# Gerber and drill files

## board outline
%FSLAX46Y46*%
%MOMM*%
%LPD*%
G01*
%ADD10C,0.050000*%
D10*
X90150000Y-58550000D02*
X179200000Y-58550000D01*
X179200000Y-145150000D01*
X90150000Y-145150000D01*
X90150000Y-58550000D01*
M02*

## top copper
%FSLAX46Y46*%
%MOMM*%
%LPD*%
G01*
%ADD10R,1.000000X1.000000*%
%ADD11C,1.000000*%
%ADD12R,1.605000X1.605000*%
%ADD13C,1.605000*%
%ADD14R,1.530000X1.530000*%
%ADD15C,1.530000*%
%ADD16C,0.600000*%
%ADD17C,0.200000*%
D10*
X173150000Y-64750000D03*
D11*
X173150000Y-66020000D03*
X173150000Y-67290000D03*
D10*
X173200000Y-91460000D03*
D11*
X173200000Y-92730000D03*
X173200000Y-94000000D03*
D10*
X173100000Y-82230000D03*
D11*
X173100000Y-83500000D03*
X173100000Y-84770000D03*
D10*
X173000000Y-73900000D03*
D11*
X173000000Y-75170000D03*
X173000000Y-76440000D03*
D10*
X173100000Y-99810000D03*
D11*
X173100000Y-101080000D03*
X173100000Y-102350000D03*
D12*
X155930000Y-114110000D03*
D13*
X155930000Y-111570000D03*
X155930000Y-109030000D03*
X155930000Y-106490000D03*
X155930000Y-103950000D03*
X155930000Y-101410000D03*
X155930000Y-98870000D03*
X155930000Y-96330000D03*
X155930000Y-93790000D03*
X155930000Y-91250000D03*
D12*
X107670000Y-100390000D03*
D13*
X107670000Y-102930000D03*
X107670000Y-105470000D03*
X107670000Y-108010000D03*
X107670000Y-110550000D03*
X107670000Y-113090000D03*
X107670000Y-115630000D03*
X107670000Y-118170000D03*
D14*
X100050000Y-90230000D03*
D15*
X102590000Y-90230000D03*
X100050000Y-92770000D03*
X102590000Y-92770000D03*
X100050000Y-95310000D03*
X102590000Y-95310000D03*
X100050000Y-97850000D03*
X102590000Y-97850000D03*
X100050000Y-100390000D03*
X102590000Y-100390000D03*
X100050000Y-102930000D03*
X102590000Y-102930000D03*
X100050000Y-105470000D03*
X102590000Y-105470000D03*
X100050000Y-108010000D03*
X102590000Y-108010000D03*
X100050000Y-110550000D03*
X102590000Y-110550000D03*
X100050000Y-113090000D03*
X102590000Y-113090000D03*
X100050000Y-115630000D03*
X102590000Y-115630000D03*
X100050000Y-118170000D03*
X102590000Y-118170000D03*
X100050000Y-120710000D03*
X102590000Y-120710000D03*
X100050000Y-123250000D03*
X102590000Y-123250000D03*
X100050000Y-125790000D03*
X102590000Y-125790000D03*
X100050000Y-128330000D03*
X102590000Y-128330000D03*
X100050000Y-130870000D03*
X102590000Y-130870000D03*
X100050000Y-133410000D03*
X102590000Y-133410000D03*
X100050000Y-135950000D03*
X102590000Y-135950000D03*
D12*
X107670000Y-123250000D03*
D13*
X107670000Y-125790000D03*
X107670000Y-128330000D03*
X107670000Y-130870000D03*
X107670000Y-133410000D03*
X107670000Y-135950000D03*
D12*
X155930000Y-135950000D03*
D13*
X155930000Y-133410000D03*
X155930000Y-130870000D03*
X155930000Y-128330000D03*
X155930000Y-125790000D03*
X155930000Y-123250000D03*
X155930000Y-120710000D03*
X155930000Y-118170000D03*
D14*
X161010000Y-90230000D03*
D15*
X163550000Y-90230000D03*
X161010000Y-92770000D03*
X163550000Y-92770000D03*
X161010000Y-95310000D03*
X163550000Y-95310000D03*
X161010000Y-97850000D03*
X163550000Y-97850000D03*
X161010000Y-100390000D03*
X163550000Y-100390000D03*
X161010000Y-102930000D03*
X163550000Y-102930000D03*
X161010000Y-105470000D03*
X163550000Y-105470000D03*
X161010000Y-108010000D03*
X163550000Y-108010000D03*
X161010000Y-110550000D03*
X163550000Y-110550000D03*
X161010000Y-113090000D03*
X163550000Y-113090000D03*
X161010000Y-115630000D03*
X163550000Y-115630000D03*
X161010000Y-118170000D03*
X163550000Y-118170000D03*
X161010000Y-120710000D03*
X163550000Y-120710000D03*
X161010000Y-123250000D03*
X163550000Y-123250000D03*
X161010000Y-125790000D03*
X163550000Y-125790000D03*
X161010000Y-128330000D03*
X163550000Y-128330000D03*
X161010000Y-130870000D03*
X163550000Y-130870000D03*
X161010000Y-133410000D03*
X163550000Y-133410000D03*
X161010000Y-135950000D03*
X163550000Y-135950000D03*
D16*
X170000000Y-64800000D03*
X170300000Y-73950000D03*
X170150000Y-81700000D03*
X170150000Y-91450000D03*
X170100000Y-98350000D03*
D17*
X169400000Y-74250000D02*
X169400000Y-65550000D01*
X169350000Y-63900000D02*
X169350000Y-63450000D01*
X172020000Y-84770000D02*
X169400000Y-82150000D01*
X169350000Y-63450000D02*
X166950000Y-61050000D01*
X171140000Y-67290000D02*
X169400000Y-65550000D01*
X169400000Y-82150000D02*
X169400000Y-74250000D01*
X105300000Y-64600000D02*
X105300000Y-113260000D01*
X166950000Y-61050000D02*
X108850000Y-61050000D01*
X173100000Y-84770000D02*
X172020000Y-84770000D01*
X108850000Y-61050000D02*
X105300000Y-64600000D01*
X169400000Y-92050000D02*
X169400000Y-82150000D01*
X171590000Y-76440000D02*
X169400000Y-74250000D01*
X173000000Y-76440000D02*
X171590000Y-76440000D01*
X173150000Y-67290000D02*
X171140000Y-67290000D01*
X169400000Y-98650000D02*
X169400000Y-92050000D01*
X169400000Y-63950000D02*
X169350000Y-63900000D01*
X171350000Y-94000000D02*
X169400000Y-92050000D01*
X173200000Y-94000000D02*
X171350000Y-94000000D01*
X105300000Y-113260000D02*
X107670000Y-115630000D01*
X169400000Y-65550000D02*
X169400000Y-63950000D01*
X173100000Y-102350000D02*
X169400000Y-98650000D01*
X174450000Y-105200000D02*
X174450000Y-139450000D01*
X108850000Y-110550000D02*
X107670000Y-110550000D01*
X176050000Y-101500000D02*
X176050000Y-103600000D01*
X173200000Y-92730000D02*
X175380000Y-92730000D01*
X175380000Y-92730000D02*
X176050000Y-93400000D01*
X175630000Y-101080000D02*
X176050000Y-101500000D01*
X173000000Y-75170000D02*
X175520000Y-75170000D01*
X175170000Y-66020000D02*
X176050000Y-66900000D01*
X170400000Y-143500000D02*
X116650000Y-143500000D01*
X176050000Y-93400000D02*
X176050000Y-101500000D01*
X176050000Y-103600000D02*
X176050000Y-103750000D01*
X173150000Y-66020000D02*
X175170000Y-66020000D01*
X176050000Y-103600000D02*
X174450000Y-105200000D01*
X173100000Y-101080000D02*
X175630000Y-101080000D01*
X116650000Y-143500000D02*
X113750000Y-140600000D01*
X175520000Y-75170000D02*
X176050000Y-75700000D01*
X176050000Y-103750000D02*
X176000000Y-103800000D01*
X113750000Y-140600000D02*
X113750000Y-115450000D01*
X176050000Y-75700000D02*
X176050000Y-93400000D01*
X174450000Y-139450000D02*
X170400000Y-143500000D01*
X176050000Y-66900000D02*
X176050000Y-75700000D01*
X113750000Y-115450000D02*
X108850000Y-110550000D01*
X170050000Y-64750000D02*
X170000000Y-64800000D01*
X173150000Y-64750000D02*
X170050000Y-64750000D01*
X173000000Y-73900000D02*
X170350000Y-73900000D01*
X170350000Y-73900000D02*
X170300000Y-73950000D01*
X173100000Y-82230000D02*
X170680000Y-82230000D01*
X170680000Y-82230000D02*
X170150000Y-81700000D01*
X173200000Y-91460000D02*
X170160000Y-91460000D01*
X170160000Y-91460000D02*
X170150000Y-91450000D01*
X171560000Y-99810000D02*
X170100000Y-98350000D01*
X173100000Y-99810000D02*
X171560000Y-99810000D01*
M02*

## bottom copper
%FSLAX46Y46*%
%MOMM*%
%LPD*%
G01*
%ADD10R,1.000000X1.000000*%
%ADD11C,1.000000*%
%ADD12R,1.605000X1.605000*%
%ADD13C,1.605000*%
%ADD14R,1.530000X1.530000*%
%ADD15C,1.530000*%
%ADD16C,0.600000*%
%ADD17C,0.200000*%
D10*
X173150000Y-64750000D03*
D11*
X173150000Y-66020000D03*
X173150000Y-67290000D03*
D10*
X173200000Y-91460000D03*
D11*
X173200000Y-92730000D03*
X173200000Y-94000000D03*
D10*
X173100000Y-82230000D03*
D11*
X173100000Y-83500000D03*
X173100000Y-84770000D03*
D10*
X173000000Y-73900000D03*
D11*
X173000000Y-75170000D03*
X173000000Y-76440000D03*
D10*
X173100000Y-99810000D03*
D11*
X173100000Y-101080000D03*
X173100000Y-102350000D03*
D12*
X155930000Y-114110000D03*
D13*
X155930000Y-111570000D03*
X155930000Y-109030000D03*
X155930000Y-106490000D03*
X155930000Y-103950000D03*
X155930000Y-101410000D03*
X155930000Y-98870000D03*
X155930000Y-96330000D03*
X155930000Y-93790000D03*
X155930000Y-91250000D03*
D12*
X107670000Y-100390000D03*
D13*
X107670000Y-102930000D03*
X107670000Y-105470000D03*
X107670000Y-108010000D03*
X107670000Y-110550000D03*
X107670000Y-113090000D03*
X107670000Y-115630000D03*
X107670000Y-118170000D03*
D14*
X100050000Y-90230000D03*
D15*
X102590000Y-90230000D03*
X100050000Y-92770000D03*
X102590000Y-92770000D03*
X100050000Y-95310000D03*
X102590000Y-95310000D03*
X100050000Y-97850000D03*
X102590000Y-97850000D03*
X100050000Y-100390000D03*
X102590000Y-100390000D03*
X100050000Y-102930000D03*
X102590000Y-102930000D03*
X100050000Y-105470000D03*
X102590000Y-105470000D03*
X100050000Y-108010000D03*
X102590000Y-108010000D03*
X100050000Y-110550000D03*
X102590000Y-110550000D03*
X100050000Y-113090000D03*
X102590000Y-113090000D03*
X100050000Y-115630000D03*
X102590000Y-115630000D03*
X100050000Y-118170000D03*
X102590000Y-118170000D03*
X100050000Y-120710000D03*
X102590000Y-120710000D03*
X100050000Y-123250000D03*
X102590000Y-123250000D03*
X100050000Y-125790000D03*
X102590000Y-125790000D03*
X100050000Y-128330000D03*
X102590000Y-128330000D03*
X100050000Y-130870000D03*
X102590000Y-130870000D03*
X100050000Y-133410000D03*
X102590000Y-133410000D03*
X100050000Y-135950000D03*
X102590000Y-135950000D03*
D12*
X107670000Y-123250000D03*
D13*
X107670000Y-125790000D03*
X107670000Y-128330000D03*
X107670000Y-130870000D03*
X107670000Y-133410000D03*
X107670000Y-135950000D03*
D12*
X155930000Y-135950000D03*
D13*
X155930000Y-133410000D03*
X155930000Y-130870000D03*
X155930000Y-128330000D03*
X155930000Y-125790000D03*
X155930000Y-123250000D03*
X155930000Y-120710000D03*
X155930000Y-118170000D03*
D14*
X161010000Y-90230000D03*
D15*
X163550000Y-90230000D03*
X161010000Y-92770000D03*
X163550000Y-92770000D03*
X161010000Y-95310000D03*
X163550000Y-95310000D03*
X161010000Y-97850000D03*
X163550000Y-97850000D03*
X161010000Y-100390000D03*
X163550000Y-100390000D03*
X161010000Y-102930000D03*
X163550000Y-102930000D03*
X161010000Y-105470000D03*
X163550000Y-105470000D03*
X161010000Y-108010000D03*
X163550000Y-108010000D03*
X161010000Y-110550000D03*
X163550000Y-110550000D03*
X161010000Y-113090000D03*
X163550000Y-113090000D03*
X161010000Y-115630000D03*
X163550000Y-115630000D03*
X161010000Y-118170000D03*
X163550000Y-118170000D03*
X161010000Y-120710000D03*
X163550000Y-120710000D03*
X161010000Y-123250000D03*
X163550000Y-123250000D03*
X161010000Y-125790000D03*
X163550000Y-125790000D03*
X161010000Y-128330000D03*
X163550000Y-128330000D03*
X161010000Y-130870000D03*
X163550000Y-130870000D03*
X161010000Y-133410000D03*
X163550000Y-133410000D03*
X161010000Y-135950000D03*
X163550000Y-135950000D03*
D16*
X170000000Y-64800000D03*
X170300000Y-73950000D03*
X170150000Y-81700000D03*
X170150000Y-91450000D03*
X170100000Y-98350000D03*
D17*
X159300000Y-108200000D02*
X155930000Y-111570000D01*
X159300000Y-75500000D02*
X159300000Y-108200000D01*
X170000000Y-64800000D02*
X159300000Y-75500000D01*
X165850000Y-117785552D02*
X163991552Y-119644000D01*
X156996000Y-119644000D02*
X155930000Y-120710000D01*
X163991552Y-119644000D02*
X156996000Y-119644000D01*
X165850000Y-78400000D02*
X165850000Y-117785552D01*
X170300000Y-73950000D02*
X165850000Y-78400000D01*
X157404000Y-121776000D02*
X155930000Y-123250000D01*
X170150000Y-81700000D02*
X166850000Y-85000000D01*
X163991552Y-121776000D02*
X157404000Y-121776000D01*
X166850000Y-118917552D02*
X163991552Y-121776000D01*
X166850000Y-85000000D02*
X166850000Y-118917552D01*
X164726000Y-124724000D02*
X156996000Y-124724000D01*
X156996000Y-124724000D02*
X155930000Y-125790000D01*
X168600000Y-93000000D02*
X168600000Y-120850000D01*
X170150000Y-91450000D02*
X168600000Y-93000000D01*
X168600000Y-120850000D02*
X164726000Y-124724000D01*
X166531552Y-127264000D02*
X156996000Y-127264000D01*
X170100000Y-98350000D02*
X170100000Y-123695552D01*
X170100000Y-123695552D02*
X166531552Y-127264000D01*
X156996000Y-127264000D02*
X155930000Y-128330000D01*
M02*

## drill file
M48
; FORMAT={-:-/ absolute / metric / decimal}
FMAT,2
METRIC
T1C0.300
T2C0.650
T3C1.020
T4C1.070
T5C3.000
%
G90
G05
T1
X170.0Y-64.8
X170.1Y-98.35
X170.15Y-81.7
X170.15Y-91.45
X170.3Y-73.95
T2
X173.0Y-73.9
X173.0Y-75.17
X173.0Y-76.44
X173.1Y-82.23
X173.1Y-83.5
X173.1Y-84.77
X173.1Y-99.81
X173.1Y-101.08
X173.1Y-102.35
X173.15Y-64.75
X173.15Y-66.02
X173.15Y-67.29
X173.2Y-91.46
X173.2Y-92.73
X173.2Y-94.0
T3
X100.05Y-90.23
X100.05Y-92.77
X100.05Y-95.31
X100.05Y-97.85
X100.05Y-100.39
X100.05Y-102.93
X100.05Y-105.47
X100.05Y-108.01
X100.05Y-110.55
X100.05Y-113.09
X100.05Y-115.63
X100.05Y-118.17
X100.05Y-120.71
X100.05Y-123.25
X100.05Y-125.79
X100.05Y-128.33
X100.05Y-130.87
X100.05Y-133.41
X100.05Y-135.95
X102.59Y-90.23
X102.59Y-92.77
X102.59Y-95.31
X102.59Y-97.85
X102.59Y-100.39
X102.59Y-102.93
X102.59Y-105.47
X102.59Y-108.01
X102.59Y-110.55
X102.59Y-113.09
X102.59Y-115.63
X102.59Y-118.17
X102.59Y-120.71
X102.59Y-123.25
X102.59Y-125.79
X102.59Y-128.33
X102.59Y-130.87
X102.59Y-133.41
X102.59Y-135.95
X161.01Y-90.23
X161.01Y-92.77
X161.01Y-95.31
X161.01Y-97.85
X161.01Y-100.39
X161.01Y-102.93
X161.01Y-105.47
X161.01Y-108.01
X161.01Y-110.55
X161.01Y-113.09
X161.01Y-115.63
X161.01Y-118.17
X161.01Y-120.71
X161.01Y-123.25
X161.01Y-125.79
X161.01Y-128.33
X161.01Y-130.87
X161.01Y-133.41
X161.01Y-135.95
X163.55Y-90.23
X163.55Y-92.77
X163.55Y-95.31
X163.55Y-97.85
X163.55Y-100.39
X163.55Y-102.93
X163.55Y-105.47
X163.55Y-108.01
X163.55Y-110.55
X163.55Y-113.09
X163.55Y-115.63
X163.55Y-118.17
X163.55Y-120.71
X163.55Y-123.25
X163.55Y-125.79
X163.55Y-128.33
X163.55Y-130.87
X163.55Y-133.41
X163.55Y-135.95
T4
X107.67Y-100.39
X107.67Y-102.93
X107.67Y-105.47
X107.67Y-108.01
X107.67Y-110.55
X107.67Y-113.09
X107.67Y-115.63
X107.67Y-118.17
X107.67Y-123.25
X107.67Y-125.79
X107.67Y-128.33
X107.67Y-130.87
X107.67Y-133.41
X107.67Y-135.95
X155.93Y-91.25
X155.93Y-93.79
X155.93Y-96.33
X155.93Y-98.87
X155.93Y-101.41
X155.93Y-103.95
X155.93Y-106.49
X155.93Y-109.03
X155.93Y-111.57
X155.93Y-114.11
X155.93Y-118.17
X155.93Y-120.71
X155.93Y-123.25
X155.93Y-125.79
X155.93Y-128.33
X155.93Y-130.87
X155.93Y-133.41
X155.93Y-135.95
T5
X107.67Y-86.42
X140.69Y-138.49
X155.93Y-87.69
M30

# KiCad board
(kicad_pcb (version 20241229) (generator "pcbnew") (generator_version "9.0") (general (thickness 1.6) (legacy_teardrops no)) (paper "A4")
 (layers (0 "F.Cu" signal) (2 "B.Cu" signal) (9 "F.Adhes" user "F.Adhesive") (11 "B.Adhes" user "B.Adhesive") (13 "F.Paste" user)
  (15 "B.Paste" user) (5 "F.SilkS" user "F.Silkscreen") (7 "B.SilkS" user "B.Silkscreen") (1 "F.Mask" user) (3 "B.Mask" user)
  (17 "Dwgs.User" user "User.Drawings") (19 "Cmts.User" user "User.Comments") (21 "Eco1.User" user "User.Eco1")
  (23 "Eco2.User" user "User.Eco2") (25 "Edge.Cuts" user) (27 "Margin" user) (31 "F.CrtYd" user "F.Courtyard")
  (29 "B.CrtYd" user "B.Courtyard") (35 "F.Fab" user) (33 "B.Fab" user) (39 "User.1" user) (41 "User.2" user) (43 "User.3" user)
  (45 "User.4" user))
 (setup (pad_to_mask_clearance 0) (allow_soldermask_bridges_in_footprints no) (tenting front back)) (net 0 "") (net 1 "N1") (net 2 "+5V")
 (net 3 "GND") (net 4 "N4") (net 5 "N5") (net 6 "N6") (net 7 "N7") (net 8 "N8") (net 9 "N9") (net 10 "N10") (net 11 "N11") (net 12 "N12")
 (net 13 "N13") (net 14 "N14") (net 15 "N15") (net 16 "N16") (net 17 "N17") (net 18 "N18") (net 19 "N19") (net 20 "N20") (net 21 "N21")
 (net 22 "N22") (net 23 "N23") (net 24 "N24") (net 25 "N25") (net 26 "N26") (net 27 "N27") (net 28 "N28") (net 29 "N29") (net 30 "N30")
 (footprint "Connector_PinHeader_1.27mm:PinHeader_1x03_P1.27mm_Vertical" (layer "F.Cu") (at 173.15 64.75)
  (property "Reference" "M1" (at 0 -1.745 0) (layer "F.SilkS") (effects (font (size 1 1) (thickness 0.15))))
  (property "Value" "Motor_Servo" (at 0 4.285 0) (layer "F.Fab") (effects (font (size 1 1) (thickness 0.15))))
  (pad "1" thru_hole rect (at 0 0) (size 1 1) (drill 0.65) (layers "*.Cu" "*.Mask") (remove_unused_layers no) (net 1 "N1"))
  (pad "2" thru_hole circle (at 0 1.27) (size 1 1) (drill 0.65) (layers "*.Cu" "*.Mask") (remove_unused_layers no) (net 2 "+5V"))
  (pad "3" thru_hole circle (at 0 2.54) (size 1 1) (drill 0.65) (layers "*.Cu" "*.Mask") (remove_unused_layers no) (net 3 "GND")))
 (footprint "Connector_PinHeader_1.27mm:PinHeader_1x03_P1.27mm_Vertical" (layer "F.Cu") (at 173.2 91.46)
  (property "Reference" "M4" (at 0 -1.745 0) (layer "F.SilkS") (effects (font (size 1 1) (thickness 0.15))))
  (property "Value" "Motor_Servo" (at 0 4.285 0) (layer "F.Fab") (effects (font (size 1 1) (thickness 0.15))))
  (pad "1" thru_hole rect (at 0 0) (size 1 1) (drill 0.65) (layers "*.Cu" "*.Mask") (remove_unused_layers no) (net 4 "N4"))
  (pad "2" thru_hole circle (at 0 1.27) (size 1 1) (drill 0.65) (layers "*.Cu" "*.Mask") (remove_unused_layers no) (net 2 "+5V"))
  (pad "3" thru_hole circle (at 0 2.54) (size 1 1) (drill 0.65) (layers "*.Cu" "*.Mask") (remove_unused_layers no) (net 3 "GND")))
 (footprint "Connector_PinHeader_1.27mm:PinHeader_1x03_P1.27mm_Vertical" (layer "F.Cu") (at 173.1 82.23)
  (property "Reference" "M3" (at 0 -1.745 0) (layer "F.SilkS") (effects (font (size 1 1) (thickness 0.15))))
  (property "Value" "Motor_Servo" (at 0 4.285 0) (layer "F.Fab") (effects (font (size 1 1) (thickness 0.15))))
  (pad "1" thru_hole rect (at 0 0) (size 1 1) (drill 0.65) (layers "*.Cu" "*.Mask") (remove_unused_layers no) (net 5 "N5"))
  (pad "2" thru_hole circle (at 0 1.27) (size 1 1) (drill 0.65) (layers "*.Cu" "*.Mask") (remove_unused_layers no) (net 2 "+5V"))
  (pad "3" thru_hole circle (at 0 2.54) (size 1 1) (drill 0.65) (layers "*.Cu" "*.Mask") (remove_unused_layers no) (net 3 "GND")))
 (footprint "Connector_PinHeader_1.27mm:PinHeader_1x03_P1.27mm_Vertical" (layer "F.Cu") (at 173 73.9)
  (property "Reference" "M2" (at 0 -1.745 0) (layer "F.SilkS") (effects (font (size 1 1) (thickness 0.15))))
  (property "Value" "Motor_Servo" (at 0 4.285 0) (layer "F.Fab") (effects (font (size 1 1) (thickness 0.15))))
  (pad "1" thru_hole rect (at 0 0) (size 1 1) (drill 0.65) (layers "*.Cu" "*.Mask") (remove_unused_layers no) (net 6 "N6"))
  (pad "2" thru_hole circle (at 0 1.27) (size 1 1) (drill 0.65) (layers "*.Cu" "*.Mask") (remove_unused_layers no) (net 2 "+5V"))
  (pad "3" thru_hole circle (at 0 2.54) (size 1 1) (drill 0.65) (layers "*.Cu" "*.Mask") (remove_unused_layers no) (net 3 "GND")))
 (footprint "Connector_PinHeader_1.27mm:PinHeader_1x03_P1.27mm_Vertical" (layer "F.Cu") (at 173.1 99.81)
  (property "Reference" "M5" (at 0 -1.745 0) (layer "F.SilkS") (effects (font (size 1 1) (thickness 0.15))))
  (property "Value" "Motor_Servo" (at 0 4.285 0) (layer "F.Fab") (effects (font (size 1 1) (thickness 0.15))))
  (pad "1" thru_hole rect (at 0 0) (size 1 1) (drill 0.65) (layers "*.Cu" "*.Mask") (remove_unused_layers no) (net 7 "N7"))
  (pad "2" thru_hole circle (at 0 1.27) (size 1 1) (drill 0.65) (layers "*.Cu" "*.Mask") (remove_unused_layers no) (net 2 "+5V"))
  (pad "3" thru_hole circle (at 0 2.54) (size 1 1) (drill 0.65) (layers "*.Cu" "*.Mask") (remove_unused_layers no) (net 3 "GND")))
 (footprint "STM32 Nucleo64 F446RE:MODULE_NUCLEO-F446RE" (layer "F.Cu") (at 131.8 99.74)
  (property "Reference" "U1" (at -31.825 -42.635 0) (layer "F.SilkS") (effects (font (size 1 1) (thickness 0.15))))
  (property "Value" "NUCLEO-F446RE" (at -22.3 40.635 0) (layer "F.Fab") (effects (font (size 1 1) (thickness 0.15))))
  (pad "" np_thru_hole circle (at -24.13 -13.32) (size 3 3) (drill 3) (layers "*.Cu" "*.Mask"))
  (pad "" np_thru_hole circle (at 8.89 38.75) (size 3 3) (drill 3) (layers "*.Cu" "*.Mask"))
  (pad "" np_thru_hole circle (at 24.13 -12.05) (size 3 3) (drill 3) (layers "*.Cu" "*.Mask"))
  (pad "CN5_1" thru_hole rect (at 24.13 14.37) (size 1.605 1.605) (drill 1.07) (layers "*.Cu" "*.Mask") (remove_unused_layers no)
   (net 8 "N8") (solder_mask_margin 0.102))
  (pad "CN5_2" thru_hole circle (at 24.13 11.83) (size 1.605 1.605) (drill 1.07) (layers "*.Cu" "*.Mask") (remove_unused_layers no)
   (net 1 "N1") (solder_mask_margin 0.102))
  (pad "CN5_3" thru_hole circle (at 24.13 9.29) (size 1.605 1.605) (drill 1.07) (layers "*.Cu" "*.Mask") (remove_unused_layers no)
   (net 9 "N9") (solder_mask_margin 0.102))
  (pad "CN5_4" thru_hole circle (at 24.13 6.75) (size 1.605 1.605) (drill 1.07) (layers "*.Cu" "*.Mask") (remove_unused_layers no)
   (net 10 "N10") (solder_mask_margin 0.102))
  (pad "CN5_5" thru_hole circle (at 24.13 4.21) (size 1.605 1.605) (drill 1.07) (layers "*.Cu" "*.Mask") (remove_unused_layers no)
   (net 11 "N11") (solder_mask_margin 0.102))
  (pad "CN5_6" thru_hole circle (at 24.13 1.67) (size 1.605 1.605) (drill 1.07) (layers "*.Cu" "*.Mask") (remove_unused_layers no)
   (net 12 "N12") (solder_mask_margin 0.102))
  (pad "CN5_7" thru_hole circle (at 24.13 -0.87) (size 1.605 1.605) (drill 1.07) (layers "*.Cu" "*.Mask") (remove_unused_layers no)
   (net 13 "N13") (solder_mask_margin 0.102))
  (pad "CN5_8" thru_hole circle (at 24.13 -3.41) (size 1.605 1.605) (drill 1.07) (layers "*.Cu" "*.Mask") (remove_unused_layers no)
   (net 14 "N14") (solder_mask_margin 0.102))
  (pad "CN5_9" thru_hole circle (at 24.13 -5.95) (size 1.605 1.605) (drill 1.07) (layers "*.Cu" "*.Mask") (remove_unused_layers no)
   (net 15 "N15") (solder_mask_margin 0.102))
  (pad "CN5_10" thru_hole circle (at 24.13 -8.49) (size 1.605 1.605) (drill 1.07) (layers "*.Cu" "*.Mask") (remove_unused_layers no)
   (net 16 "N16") (solder_mask_margin 0.102))
  (pad "CN6_1" thru_hole rect (at -24.13 0.65) (size 1.605 1.605) (drill 1.07) (layers "*.Cu" "*.Mask") (remove_unused_layers no)
   (solder_mask_margin 0.102))
  (pad "CN6_2" thru_hole circle (at -24.13 3.19) (size 1.605 1.605) (drill 1.07) (layers "*.Cu" "*.Mask") (remove_unused_layers no)
   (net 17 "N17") (solder_mask_margin 0.102))
  (pad "CN6_3" thru_hole circle (at -24.13 5.73) (size 1.605 1.605) (drill 1.07) (layers "*.Cu" "*.Mask") (remove_unused_layers no)
   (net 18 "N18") (solder_mask_margin 0.102))
  (pad "CN6_4" thru_hole circle (at -24.13 8.27) (size 1.605 1.605) (drill 1.07) (layers "*.Cu" "*.Mask") (remove_unused_layers no)
   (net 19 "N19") (solder_mask_margin 0.102))
  (pad "CN6_5" thru_hole circle (at -24.13 10.81) (size 1.605 1.605) (drill 1.07) (layers "*.Cu" "*.Mask") (remove_unused_layers no)
   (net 2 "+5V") (solder_mask_margin 0.102))
  (pad "CN6_6" thru_hole circle (at -24.13 13.35) (size 1.605 1.605) (drill 1.07) (layers "*.Cu" "*.Mask") (remove_unused_layers no)
   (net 3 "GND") (solder_mask_margin 0.102))
  (pad "CN6_7" thru_hole circle (at -24.13 15.89) (size 1.605 1.605) (drill 1.07) (layers "*.Cu" "*.Mask") (remove_unused_layers no)
   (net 3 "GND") (solder_mask_margin 0.102))
  (pad "CN6_8" thru_hole circle (at -24.13 18.43) (size 1.605 1.605) (drill 1.07) (layers "*.Cu" "*.Mask") (remove_unused_layers no)
   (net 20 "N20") (solder_mask_margin 0.102))
  (pad "CN7_1" thru_hole rect (at -31.75 -9.51) (size 1.53 1.53) (drill 1.02) (layers "*.Cu" "*.Mask") (remove_unused_layers no)
   (solder_mask_margin 0.102))
  (pad "CN7_2" thru_hole circle (at -29.21 -9.51) (size 1.53 1.53) (drill 1.02) (layers "*.Cu" "*.Mask") (remove_unused_layers no)
   (solder_mask_margin 0.102))
  (pad "CN7_3" thru_hole circle (at -31.75 -6.97) (size 1.53 1.53) (drill 1.02) (layers "*.Cu" "*.Mask") (remove_unused_layers no)
   (solder_mask_margin 0.102))
  (pad "CN7_4" thru_hole circle (at -29.21 -6.97) (size 1.53 1.53) (drill 1.02) (layers "*.Cu" "*.Mask") (remove_unused_layers no)
   (solder_mask_margin 0.102))
  (pad "CN7_5" thru_hole circle (at -31.75 -4.43) (size 1.53 1.53) (drill 1.02) (layers "*.Cu" "*.Mask") (remove_unused_layers no)
   (solder_mask_margin 0.102))
  (pad "CN7_6" thru_hole circle (at -29.21 -4.43) (size 1.53 1.53) (drill 1.02) (layers "*.Cu" "*.Mask") (remove_unused_layers no)
   (solder_mask_margin 0.102))
  (pad "CN7_7" thru_hole circle (at -31.75 -1.89) (size 1.53 1.53) (drill 1.02) (layers "*.Cu" "*.Mask") (remove_unused_layers no)
   (solder_mask_margin 0.102))
  (pad "CN7_8" thru_hole circle (at -29.21 -1.89) (size 1.53 1.53) (drill 1.02) (layers "*.Cu" "*.Mask") (remove_unused_layers no)
   (solder_mask_margin 0.102))
  (pad "CN7_9" thru_hole circle (at -31.75 0.65) (size 1.53 1.53) (drill 1.02) (layers "*.Cu" "*.Mask") (remove_unused_layers no)
   (solder_mask_margin 0.102))
  (pad "CN7_10" thru_hole circle (at -29.21 0.65) (size 1.53 1.53) (drill 1.02) (layers "*.Cu" "*.Mask") (remove_unused_layers no)
   (solder_mask_margin 0.102))
  (pad "CN7_11" thru_hole circle (at -31.75 3.19) (size 1.53 1.53) (drill 1.02) (layers "*.Cu" "*.Mask") (remove_unused_layers no)
   (solder_mask_margin 0.102))
  (pad "CN7_12" thru_hole circle (at -29.21 3.19) (size 1.53 1.53) (drill 1.02) (layers "*.Cu" "*.Mask") (remove_unused_layers no)
   (solder_mask_margin 0.102))
  (pad "CN7_13" thru_hole circle (at -31.75 5.73) (size 1.53 1.53) (drill 1.02) (layers "*.Cu" "*.Mask") (remove_unused_layers no)
   (solder_mask_margin 0.102))
  (pad "CN7_14" thru_hole circle (at -29.21 5.73) (size 1.53 1.53) (drill 1.02) (layers "*.Cu" "*.Mask") (remove_unused_layers no)
   (solder_mask_margin 0.102))
  (pad "CN7_15" thru_hole circle (at -31.75 8.27) (size 1.53 1.53) (drill 1.02) (layers "*.Cu" "*.Mask") (remove_unused_layers no)
   (solder_mask_margin 0.102))
  (pad "CN7_16" thru_hole circle (at -29.21 8.27) (size 1.53 1.53) (drill 1.02) (layers "*.Cu" "*.Mask") (remove_unused_layers no)
   (solder_mask_margin 0.102))
  (pad "CN7_17" thru_hole circle (at -31.75 10.81) (size 1.53 1.53) (drill 1.02) (layers "*.Cu" "*.Mask") (remove_unused_layers no)
   (solder_mask_margin 0.102))
  (pad "CN7_18" thru_hole circle (at -29.21 10.81) (size 1.53 1.53) (drill 1.02) (layers "*.Cu" "*.Mask") (remove_unused_layers no)
   (solder_mask_margin 0.102))
  (pad "CN7_19" thru_hole circle (at -31.75 13.35) (size 1.53 1.53) (drill 1.02) (layers "*.Cu" "*.Mask") (remove_unused_layers no)
   (solder_mask_margin 0.102))
  (pad "CN7_20" thru_hole circle (at -29.21 13.35) (size 1.53 1.53) (drill 1.02) (layers "*.Cu" "*.Mask") (remove_unused_layers no)
   (solder_mask_margin 0.102))
  (pad "CN7_21" thru_hole circle (at -31.75 15.89) (size 1.53 1.53) (drill 1.02) (layers "*.Cu" "*.Mask") (remove_unused_layers no)
   (solder_mask_margin 0.102))
  (pad "CN7_22" thru_hole circle (at -29.21 15.89) (size 1.53 1.53) (drill 1.02) (layers "*.Cu" "*.Mask") (remove_unused_layers no)
   (solder_mask_margin 0.102))
  (pad "CN7_23" thru_hole circle (at -31.75 18.43) (size 1.53 1.53) (drill 1.02) (layers "*.Cu" "*.Mask") (remove_unused_layers no)
   (solder_mask_margin 0.102))
  (pad "CN7_24" thru_hole circle (at -29.21 18.43) (size 1.53 1.53) (drill 1.02) (layers "*.Cu" "*.Mask") (remove_unused_layers no)
   (solder_mask_margin 0.102))
  (pad "CN7_25" thru_hole circle (at -31.75 20.97) (size 1.53 1.53) (drill 1.02) (layers "*.Cu" "*.Mask") (remove_unused_layers no)
   (solder_mask_margin 0.102))
  (pad "CN7_26" thru_hole circle (at -29.21 20.97) (size 1.53 1.53) (drill 1.02) (layers "*.Cu" "*.Mask") (remove_unused_layers no)
   (solder_mask_margin 0.102))
  (pad "CN7_27" thru_hole circle (at -31.75 23.51) (size 1.53 1.53) (drill 1.02) (layers "*.Cu" "*.Mask") (remove_unused_layers no)
   (solder_mask_margin 0.102))
  (pad "CN7_28" thru_hole circle (at -29.21 23.51) (size 1.53 1.53) (drill 1.02) (layers "*.Cu" "*.Mask") (remove_unused_layers no)
   (solder_mask_margin 0.102))
  (pad "CN7_29" thru_hole circle (at -31.75 26.05) (size 1.53 1.53) (drill 1.02) (layers "*.Cu" "*.Mask") (remove_unused_layers no)
   (solder_mask_margin 0.102))
  (pad "CN7_30" thru_hole circle (at -29.21 26.05) (size 1.53 1.53) (drill 1.02) (layers "*.Cu" "*.Mask") (remove_unused_layers no)
   (solder_mask_margin 0.102))
  (pad "CN7_31" thru_hole circle (at -31.75 28.59) (size 1.53 1.53) (drill 1.02) (layers "*.Cu" "*.Mask") (remove_unused_layers no)
   (solder_mask_margin 0.102))
  (pad "CN7_32" thru_hole circle (at -29.21 28.59) (size 1.53 1.53) (drill 1.02) (layers "*.Cu" "*.Mask") (remove_unused_layers no)
   (solder_mask_margin 0.102))
  (pad "CN7_33" thru_hole circle (at -31.75 31.13) (size 1.53 1.53) (drill 1.02) (layers "*.Cu" "*.Mask") (remove_unused_layers no)
   (solder_mask_margin 0.102))
  (pad "CN7_34" thru_hole circle (at -29.21 31.13) (size 1.53 1.53) (drill 1.02) (layers "*.Cu" "*.Mask") (remove_unused_layers no)
   (solder_mask_margin 0.102))
  (pad "CN7_35" thru_hole circle (at -31.75 33.67) (size 1.53 1.53) (drill 1.02) (layers "*.Cu" "*.Mask") (remove_unused_layers no)
   (solder_mask_margin 0.102))
  (pad "CN7_36" thru_hole circle (at -29.21 33.67) (size 1.53 1.53) (drill 1.02) (layers "*.Cu" "*.Mask") (remove_unused_layers no)
   (solder_mask_margin 0.102))
  (pad "CN7_37" thru_hole circle (at -31.75 36.21) (size 1.53 1.53) (drill 1.02) (layers "*.Cu" "*.Mask") (remove_unused_layers no)
   (solder_mask_margin 0.102))
  (pad "CN7_38" thru_hole circle (at -29.21 36.21) (size 1.53 1.53) (drill 1.02) (layers "*.Cu" "*.Mask") (remove_unused_layers no)
   (solder_mask_margin 0.102))
  (pad "CN8_1" thru_hole rect (at -24.13 23.51) (size 1.605 1.605) (drill 1.07) (layers "*.Cu" "*.Mask") (remove_unused_layers no)
   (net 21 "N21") (solder_mask_margin 0.102))
  (pad "CN8_2" thru_hole circle (at -24.13 26.05) (size 1.605 1.605) (drill 1.07) (layers "*.Cu" "*.Mask") (remove_unused_layers no)
   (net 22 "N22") (solder_mask_margin 0.102))
  (pad "CN8_3" thru_hole circle (at -24.13 28.59) (size 1.605 1.605) (drill 1.07) (layers "*.Cu" "*.Mask") (remove_unused_layers no)
   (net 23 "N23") (solder_mask_margin 0.102))
  (pad "CN8_4" thru_hole circle (at -24.13 31.13) (size 1.605 1.605) (drill 1.07) (layers "*.Cu" "*.Mask") (remove_unused_layers no)
   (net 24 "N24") (solder_mask_margin 0.102))
  (pad "CN8_5" thru_hole circle (at -24.13 33.67) (size 1.605 1.605) (drill 1.07) (layers "*.Cu" "*.Mask") (remove_unused_layers no)
   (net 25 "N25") (solder_mask_margin 0.102))
  (pad "CN8_6" thru_hole circle (at -24.13 36.21) (size 1.605 1.605) (drill 1.07) (layers "*.Cu" "*.Mask") (remove_unused_layers no)
   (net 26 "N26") (solder_mask_margin 0.102))
  (pad "CN9_1" thru_hole rect (at 24.13 36.21) (size 1.605 1.605) (drill 1.07) (layers "*.Cu" "*.Mask") (remove_unused_layers no)
   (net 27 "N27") (solder_mask_margin 0.102))
  (pad "CN9_2" thru_hole circle (at 24.13 33.67) (size 1.605 1.605) (drill 1.07) (layers "*.Cu" "*.Mask") (remove_unused_layers no)
   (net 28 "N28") (solder_mask_margin 0.102))
  (pad "CN9_3" thru_hole circle (at 24.13 31.13) (size 1.605 1.605) (drill 1.07) (layers "*.Cu" "*.Mask") (remove_unused_layers no)
   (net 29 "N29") (solder_mask_margin 0.102))
  (pad "CN9_4" thru_hole circle (at 24.13 28.59) (size 1.605 1.605) (drill 1.07) (layers "*.Cu" "*.Mask") (remove_unused_layers no)
   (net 7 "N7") (solder_mask_margin 0.102))
  (pad "CN9_5" thru_hole circle (at 24.13 26.05) (size 1.605 1.605) (drill 1.07) (layers "*.Cu" "*.Mask") (remove_unused_layers no)
   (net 4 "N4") (solder_mask_margin 0.102))
  (pad "CN9_6" thru_hole circle (at 24.13 23.51) (size 1.605 1.605) (drill 1.07) (layers "*.Cu" "*.Mask") (remove_unused_layers no)
   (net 5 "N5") (solder_mask_margin 0.102))
  (pad "CN9_7" thru_hole circle (at 24.13 20.97) (size 1.605 1.605) (drill 1.07) (layers "*.Cu" "*.Mask") (remove_unused_layers no)
   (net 6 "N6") (solder_mask_margin 0.102))
  (pad "CN9_8" thru_hole circle (at 24.13 18.43) (size 1.605 1.605) (drill 1.07) (layers "*.Cu" "*.Mask") (remove_unused_layers no)
   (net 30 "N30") (solder_mask_margin 0.102))
  (pad "CN10_1" thru_hole rect (at 29.21 -9.51) (size 1.53 1.53) (drill 1.02) (layers "*.Cu" "*.Mask") (remove_unused_layers no)
   (solder_mask_margin 0.102))
  (pad "CN10_2" thru_hole circle (at 31.75 -9.51) (size 1.53 1.53) (drill 1.02) (layers "*.Cu" "*.Mask") (remove_unused_layers no)
   (solder_mask_margin 0.102))
  (pad "CN10_3" thru_hole circle (at 29.21 -6.97) (size 1.53 1.53) (drill 1.02) (layers "*.Cu" "*.Mask") (remove_unused_layers no)
   (solder_mask_margin 0.102))
  (pad "CN10_4" thru_hole circle (at 31.75 -6.97) (size 1.53 1.53) (drill 1.02) (layers "*.Cu" "*.Mask") (remove_unused_layers no)
   (solder_mask_margin 0.102))
  (pad "CN10_5" thru_hole circle (at 29.21 -4.43) (size 1.53 1.53) (drill 1.02) (layers "*.Cu" "*.Mask") (remove_unused_layers no)
   (solder_mask_margin 0.102))
  (pad "CN10_6" thru_hole circle (at 31.75 -4.43) (size 1.53 1.53) (drill 1.02) (layers "*.Cu" "*.Mask") (remove_unused_layers no)
   (solder_mask_margin 0.102))
  (pad "CN10_7" thru_hole circle (at 29.21 -1.89) (size 1.53 1.53) (drill 1.02) (layers "*.Cu" "*.Mask") (remove_unused_layers no)
   (solder_mask_margin 0.102))
  (pad "CN10_8" thru_hole circle (at 31.75 -1.89) (size 1.53 1.53) (drill 1.02) (layers "*.Cu" "*.Mask") (remove_unused_layers no)
   (solder_mask_margin 0.102))
  (pad "CN10_9" thru_hole circle (at 29.21 0.65) (size 1.53 1.53) (drill 1.02) (layers "*.Cu" "*.Mask") (remove_unused_layers no)
   (solder_mask_margin 0.102))
  (pad "CN10_10" thru_hole circle (at 31.75 0.65) (size 1.53 1.53) (drill 1.02) (layers "*.Cu" "*.Mask") (remove_unused_layers no)
   (solder_mask_margin 0.102))
  (pad "CN10_11" thru_hole circle (at 29.21 3.19) (size 1.53 1.53) (drill 1.02) (layers "*.Cu" "*.Mask") (remove_unused_layers no)
   (solder_mask_margin 0.102))
  (pad "CN10_12" thru_hole circle (at 31.75 3.19) (size 1.53 1.53) (drill 1.02) (layers "*.Cu" "*.Mask") (remove_unused_layers no)
   (solder_mask_margin 0.102))
  (pad "CN10_13" thru_hole circle (at 29.21 5.73) (size 1.53 1.53) (drill 1.02) (layers "*.Cu" "*.Mask") (remove_unused_layers no)
   (solder_mask_margin 0.102))
  (pad "CN10_14" thru_hole circle (at 31.75 5.73) (size 1.53 1.53) (drill 1.02) (layers "*.Cu" "*.Mask") (remove_unused_layers no)
   (solder_mask_margin 0.102))
  (pad "CN10_15" thru_hole circle (at 29.21 8.27) (size 1.53 1.53) (drill 1.02) (layers "*.Cu" "*.Mask") (remove_unused_layers no)
   (solder_mask_margin 0.102))
  (pad "CN10_16" thru_hole circle (at 31.75 8.27) (size 1.53 1.53) (drill 1.02) (layers "*.Cu" "*.Mask") (remove_unused_layers no)
   (solder_mask_margin 0.102))
  (pad "CN10_17" thru_hole circle (at 29.21 10.81) (size 1.53 1.53) (drill 1.02) (layers "*.Cu" "*.Mask") (remove_unused_layers no)
   (solder_mask_margin 0.102))
  (pad "CN10_18" thru_hole circle (at 31.75 10.81) (size 1.53 1.53) (drill 1.02) (layers "*.Cu" "*.Mask") (remove_unused_layers no)
   (solder_mask_margin 0.102))
  (pad "CN10_19" thru_hole circle (at 29.21 13.35) (size 1.53 1.53) (drill 1.02) (layers "*.Cu" "*.Mask") (remove_unused_layers no)
   (solder_mask_margin 0.102))
  (pad "CN10_20" thru_hole circle (at 31.75 13.35) (size 1.53 1.53) (drill 1.02) (layers "*.Cu" "*.Mask") (remove_unused_layers no)
   (solder_mask_margin 0.102))
  (pad "CN10_21" thru_hole circle (at 29.21 15.89) (size 1.53 1.53) (drill 1.02) (layers "*.Cu" "*.Mask") (remove_unused_layers no)
   (solder_mask_margin 0.102))
  (pad "CN10_22" thru_hole circle (at 31.75 15.89) (size 1.53 1.53) (drill 1.02) (layers "*.Cu" "*.Mask") (remove_unused_layers no)
   (solder_mask_margin 0.102))
  (pad "CN10_23" thru_hole circle (at 29.21 18.43) (size 1.53 1.53) (drill 1.02) (layers "*.Cu" "*.Mask") (remove_unused_layers no)
   (solder_mask_margin 0.102))
  (pad "CN10_24" thru_hole circle (at 31.75 18.43) (size 1.53 1.53) (drill 1.02) (layers "*.Cu" "*.Mask") (remove_unused_layers no)
   (solder_mask_margin 0.102))
  (pad "CN10_25" thru_hole circle (at 29.21 20.97) (size 1.53 1.53) (drill 1.02) (layers "*.Cu" "*.Mask") (remove_unused_layers no)
   (solder_mask_margin 0.102))
  (pad "CN10_26" thru_hole circle (at 31.75 20.97) (size 1.53 1.53) (drill 1.02) (layers "*.Cu" "*.Mask") (remove_unused_layers no)
   (solder_mask_margin 0.102))
  (pad "CN10_27" thru_hole circle (at 29.21 23.51) (size 1.53 1.53) (drill 1.02) (layers "*.Cu" "*.Mask") (remove_unused_layers no)
   (solder_mask_margin 0.102))
  (pad "CN10_28" thru_hole circle (at 31.75 23.51) (size 1.53 1.53) (drill 1.02) (layers "*.Cu" "*.Mask") (remove_unused_layers no)
   (solder_mask_margin 0.102))
  (pad "CN10_29" thru_hole circle (at 29.21 26.05) (size 1.53 1.53) (drill 1.02) (layers "*.Cu" "*.Mask") (remove_unused_layers no)
   (solder_mask_margin 0.102))
  (pad "CN10_30" thru_hole circle (at 31.75 26.05) (size 1.53 1.53) (drill 1.02) (layers "*.Cu" "*.Mask") (remove_unused_layers no)
   (solder_mask_margin 0.102))
  (pad "CN10_31" thru_hole circle (at 29.21 28.59) (size 1.53 1.53) (drill 1.02) (layers "*.Cu" "*.Mask") (remove_unused_layers no)
   (solder_mask_margin 0.102))
  (pad "CN10_32" thru_hole circle (at 31.75 28.59) (size 1.53 1.53) (drill 1.02) (layers "*.Cu" "*.Mask") (remove_unused_layers no)
   (solder_mask_margin 0.102))
  (pad "CN10_33" thru_hole circle (at 29.21 31.13) (size 1.53 1.53) (drill 1.02) (layers "*.Cu" "*.Mask") (remove_unused_layers no)
   (solder_mask_margin 0.102))
  (pad "CN10_34" thru_hole circle (at 31.75 31.13) (size 1.53 1.53) (drill 1.02) (layers "*.Cu" "*.Mask") (remove_unused_layers no)
   (solder_mask_margin 0.102))
  (pad "CN10_35" thru_hole circle (at 29.21 33.67) (size 1.53 1.53) (drill 1.02) (layers "*.Cu" "*.Mask") (remove_unused_layers no)
   (solder_mask_margin 0.102))
  (pad "CN10_36" thru_hole circle (at 31.75 33.67) (size 1.53 1.53) (drill 1.02) (layers "*.Cu" "*.Mask") (remove_unused_layers no)
   (solder_mask_margin 0.102))
  (pad "CN10_37" thru_hole circle (at 29.21 36.21) (size 1.53 1.53) (drill 1.02) (layers "*.Cu" "*.Mask") (remove_unused_layers no)
   (solder_mask_margin 0.102))
  (pad "CN10_38" thru_hole circle (at 31.75 36.21) (size 1.53 1.53) (drill 1.02) (layers "*.Cu" "*.Mask") (remove_unused_layers no)
   (solder_mask_margin 0.102)))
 (gr_rect (start 90.15 58.55) (end 179.2 145.15) (stroke (width 0.05) (type default)) (fill no) (layer "Edge.Cuts"))
 (segment (start 169.4 74.25) (end 169.4 65.55) (width 0.2) (layer "F.Cu") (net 3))
 (segment (start 169.35 63.9) (end 169.35 63.45) (width 0.2) (layer "F.Cu") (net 3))
 (segment (start 172.02 84.77) (end 169.4 82.15) (width 0.2) (layer "F.Cu") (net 3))
 (segment (start 169.35 63.45) (end 166.95 61.05) (width 0.2) (layer "F.Cu") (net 3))
 (segment (start 171.14 67.29) (end 169.4 65.55) (width 0.2) (layer "F.Cu") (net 3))
 (segment (start 169.4 82.15) (end 169.4 74.25) (width 0.2) (layer "F.Cu") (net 3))
 (segment (start 105.3 64.6) (end 105.3 113.26) (width 0.2) (layer "F.Cu") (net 3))
 (segment (start 166.95 61.05) (end 108.85 61.05) (width 0.2) (layer "F.Cu") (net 3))
 (segment (start 173.1 84.77) (end 172.02 84.77) (width 0.2) (layer "F.Cu") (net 3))
 (segment (start 108.85 61.05) (end 105.3 64.6) (width 0.2) (layer "F.Cu") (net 3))
 (segment (start 169.4 92.05) (end 169.4 82.15) (width 0.2) (layer "F.Cu") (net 3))
 (segment (start 171.59 76.44) (end 169.4 74.25) (width 0.2) (layer "F.Cu") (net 3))
 (segment (start 173 76.44) (end 171.59 76.44) (width 0.2) (layer "F.Cu") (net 3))
 (segment (start 173.15 67.29) (end 171.14 67.29) (width 0.2) (layer "F.Cu") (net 3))
 (segment (start 169.4 98.65) (end 169.4 92.05) (width 0.2) (layer "F.Cu") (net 3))
 (segment (start 169.4 63.95) (end 169.35 63.9) (width 0.2) (layer "F.Cu") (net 3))
 (segment (start 171.35 94) (end 169.4 92.05) (width 0.2) (layer "F.Cu") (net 3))
 (segment (start 173.2 94) (end 171.35 94) (width 0.2) (layer "F.Cu") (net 3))
 (segment (start 105.3 113.26) (end 107.67 115.63) (width 0.2) (layer "F.Cu") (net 3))
 (segment (start 169.4 65.55) (end 169.4 63.95) (width 0.2) (layer "F.Cu") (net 3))
 (segment (start 173.1 102.35) (end 169.4 98.65) (width 0.2) (layer "F.Cu") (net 3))
 (segment (start 174.45 105.2) (end 174.45 139.45) (width 0.2) (layer "F.Cu") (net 2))
 (segment (start 108.85 110.55) (end 107.67 110.55) (width 0.2) (layer "F.Cu") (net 2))
 (segment (start 176.05 101.5) (end 176.05 103.6) (width 0.2) (layer "F.Cu") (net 2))
 (segment (start 173.2 92.73) (end 175.38 92.73) (width 0.2) (layer "F.Cu") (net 2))
 (segment (start 175.38 92.73) (end 176.05 93.4) (width 0.2) (layer "F.Cu") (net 2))
 (segment (start 175.63 101.08) (end 176.05 101.5) (width 0.2) (layer "F.Cu") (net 2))
 (segment (start 173 75.17) (end 175.52 75.17) (width 0.2) (layer "F.Cu") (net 2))
 (segment (start 175.17 66.02) (end 176.05 66.9) (width 0.2) (layer "F.Cu") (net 2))
 (segment (start 170.4 143.5) (end 116.65 143.5) (width 0.2) (layer "F.Cu") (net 2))
 (segment (start 176.05 93.4) (end 176.05 101.5) (width 0.2) (layer "F.Cu") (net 2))
 (segment (start 176.05 103.6) (end 176.05 103.75) (width 0.2) (layer "F.Cu") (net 2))
 (segment (start 173.15 66.02) (end 175.17 66.02) (width 0.2) (layer "F.Cu") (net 2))
 (segment (start 176.05 103.6) (end 174.45 105.2) (width 0.2) (layer "F.Cu") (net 2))
 (segment (start 173.1 101.08) (end 175.63 101.08) (width 0.2) (layer "F.Cu") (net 2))
 (segment (start 116.65 143.5) (end 113.75 140.6) (width 0.2) (layer "F.Cu") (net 2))
 (segment (start 175.52 75.17) (end 176.05 75.7) (width 0.2) (layer "F.Cu") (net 2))
 (segment (start 176.05 103.75) (end 176 103.8) (width 0.2) (layer "F.Cu") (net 2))
 (segment (start 113.75 140.6) (end 113.75 115.45) (width 0.2) (layer "F.Cu") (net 2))
 (segment (start 176.05 75.7) (end 176.05 93.4) (width 0.2) (layer "F.Cu") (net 2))
 (segment (start 174.45 139.45) (end 170.4 143.5) (width 0.2) (layer "F.Cu") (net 2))
 (segment (start 176.05 66.9) (end 176.05 75.7) (width 0.2) (layer "F.Cu") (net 2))
 (segment (start 113.75 115.45) (end 108.85 110.55) (width 0.2) (layer "F.Cu") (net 2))
 (segment (start 170.05 64.75) (end 170 64.8) (width 0.2) (layer "F.Cu") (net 1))
 (segment (start 173.15 64.75) (end 170.05 64.75) (width 0.2) (layer "F.Cu") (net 1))
 (via (at 170 64.8) (size 0.6) (drill 0.3) (layers "F.Cu" "B.Cu") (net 1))
 (segment (start 159.3 108.2) (end 155.93 111.57) (width 0.2) (layer "B.Cu") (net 1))
 (segment (start 159.3 75.5) (end 159.3 108.2) (width 0.2) (layer "B.Cu") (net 1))
 (segment (start 170 64.8) (end 159.3 75.5) (width 0.2) (layer "B.Cu") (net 1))
 (segment (start 173 73.9) (end 170.35 73.9) (width 0.2) (layer "F.Cu") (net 6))
 (segment (start 170.35 73.9) (end 170.3 73.95) (width 0.2) (layer "F.Cu") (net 6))
 (via (at 170.3 73.95) (size 0.6) (drill 0.3) (layers "F.Cu" "B.Cu") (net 6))
 (segment (start 165.85 117.785552) (end 163.991552 119.644) (width 0.2) (layer "B.Cu") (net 6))
 (segment (start 156.996 119.644) (end 155.93 120.71) (width 0.2) (layer "B.Cu") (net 6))
 (segment (start 163.991552 119.644) (end 156.996 119.644) (width 0.2) (layer "B.Cu") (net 6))
 (segment (start 165.85 78.4) (end 165.85 117.785552) (width 0.2) (layer "B.Cu") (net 6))
 (segment (start 170.3 73.95) (end 165.85 78.4) (width 0.2) (layer "B.Cu") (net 6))
 (segment (start 173.1 82.23) (end 170.68 82.23) (width 0.2) (layer "F.Cu") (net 5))
 (segment (start 170.68 82.23) (end 170.15 81.7) (width 0.2) (layer "F.Cu") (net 5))
 (via (at 170.15 81.7) (size 0.6) (drill 0.3) (layers "F.Cu" "B.Cu") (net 5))
 (segment (start 157.404 121.776) (end 155.93 123.25) (width 0.2) (layer "B.Cu") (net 5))
 (segment (start 170.15 81.7) (end 166.85 85) (width 0.2) (layer "B.Cu") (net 5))
 (segment (start 163.991552 121.776) (end 157.404 121.776) (width 0.2) (layer "B.Cu") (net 5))
 (segment (start 166.85 118.917552) (end 163.991552 121.776) (width 0.2) (layer "B.Cu") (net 5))
 (segment (start 166.85 85) (end 166.85 118.917552) (width 0.2) (layer "B.Cu") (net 5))
 (segment (start 173.2 91.46) (end 170.16 91.46) (width 0.2) (layer "F.Cu") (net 4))
 (segment (start 170.16 91.46) (end 170.15 91.45) (width 0.2) (layer "F.Cu") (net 4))
 (via (at 170.15 91.45) (size 0.6) (drill 0.3) (layers "F.Cu" "B.Cu") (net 4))
 (segment (start 164.726 124.724) (end 156.996 124.724) (width 0.2) (layer "B.Cu") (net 4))
 (segment (start 156.996 124.724) (end 155.93 125.79) (width 0.2) (layer "B.Cu") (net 4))
 (segment (start 168.6 93) (end 168.6 120.85) (width 0.2) (layer "B.Cu") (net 4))
 (segment (start 170.15 91.45) (end 168.6 93) (width 0.2) (layer "B.Cu") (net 4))
 (segment (start 168.6 120.85) (end 164.726 124.724) (width 0.2) (layer "B.Cu") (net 4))
 (segment (start 171.56 99.81) (end 170.1 98.35) (width 0.2) (layer "F.Cu") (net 7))
 (segment (start 173.1 99.81) (end 171.56 99.81) (width 0.2) (layer "F.Cu") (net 7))
 (via (at 170.1 98.35) (size 0.6) (drill 0.3) (layers "F.Cu" "B.Cu") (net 7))
 (segment (start 166.531552 127.264) (end 156.996 127.264) (width 0.2) (layer "B.Cu") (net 7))
 (segment (start 170.1 98.35) (end 170.1 123.695552) (width 0.2) (layer "B.Cu") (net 7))
 (segment (start 170.1 123.695552) (end 166.531552 127.264) (width 0.2) (layer "B.Cu") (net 7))
 (segment (start 156.996 127.264) (end 155.93 128.33) (width 0.2) (layer "B.Cu") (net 7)))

